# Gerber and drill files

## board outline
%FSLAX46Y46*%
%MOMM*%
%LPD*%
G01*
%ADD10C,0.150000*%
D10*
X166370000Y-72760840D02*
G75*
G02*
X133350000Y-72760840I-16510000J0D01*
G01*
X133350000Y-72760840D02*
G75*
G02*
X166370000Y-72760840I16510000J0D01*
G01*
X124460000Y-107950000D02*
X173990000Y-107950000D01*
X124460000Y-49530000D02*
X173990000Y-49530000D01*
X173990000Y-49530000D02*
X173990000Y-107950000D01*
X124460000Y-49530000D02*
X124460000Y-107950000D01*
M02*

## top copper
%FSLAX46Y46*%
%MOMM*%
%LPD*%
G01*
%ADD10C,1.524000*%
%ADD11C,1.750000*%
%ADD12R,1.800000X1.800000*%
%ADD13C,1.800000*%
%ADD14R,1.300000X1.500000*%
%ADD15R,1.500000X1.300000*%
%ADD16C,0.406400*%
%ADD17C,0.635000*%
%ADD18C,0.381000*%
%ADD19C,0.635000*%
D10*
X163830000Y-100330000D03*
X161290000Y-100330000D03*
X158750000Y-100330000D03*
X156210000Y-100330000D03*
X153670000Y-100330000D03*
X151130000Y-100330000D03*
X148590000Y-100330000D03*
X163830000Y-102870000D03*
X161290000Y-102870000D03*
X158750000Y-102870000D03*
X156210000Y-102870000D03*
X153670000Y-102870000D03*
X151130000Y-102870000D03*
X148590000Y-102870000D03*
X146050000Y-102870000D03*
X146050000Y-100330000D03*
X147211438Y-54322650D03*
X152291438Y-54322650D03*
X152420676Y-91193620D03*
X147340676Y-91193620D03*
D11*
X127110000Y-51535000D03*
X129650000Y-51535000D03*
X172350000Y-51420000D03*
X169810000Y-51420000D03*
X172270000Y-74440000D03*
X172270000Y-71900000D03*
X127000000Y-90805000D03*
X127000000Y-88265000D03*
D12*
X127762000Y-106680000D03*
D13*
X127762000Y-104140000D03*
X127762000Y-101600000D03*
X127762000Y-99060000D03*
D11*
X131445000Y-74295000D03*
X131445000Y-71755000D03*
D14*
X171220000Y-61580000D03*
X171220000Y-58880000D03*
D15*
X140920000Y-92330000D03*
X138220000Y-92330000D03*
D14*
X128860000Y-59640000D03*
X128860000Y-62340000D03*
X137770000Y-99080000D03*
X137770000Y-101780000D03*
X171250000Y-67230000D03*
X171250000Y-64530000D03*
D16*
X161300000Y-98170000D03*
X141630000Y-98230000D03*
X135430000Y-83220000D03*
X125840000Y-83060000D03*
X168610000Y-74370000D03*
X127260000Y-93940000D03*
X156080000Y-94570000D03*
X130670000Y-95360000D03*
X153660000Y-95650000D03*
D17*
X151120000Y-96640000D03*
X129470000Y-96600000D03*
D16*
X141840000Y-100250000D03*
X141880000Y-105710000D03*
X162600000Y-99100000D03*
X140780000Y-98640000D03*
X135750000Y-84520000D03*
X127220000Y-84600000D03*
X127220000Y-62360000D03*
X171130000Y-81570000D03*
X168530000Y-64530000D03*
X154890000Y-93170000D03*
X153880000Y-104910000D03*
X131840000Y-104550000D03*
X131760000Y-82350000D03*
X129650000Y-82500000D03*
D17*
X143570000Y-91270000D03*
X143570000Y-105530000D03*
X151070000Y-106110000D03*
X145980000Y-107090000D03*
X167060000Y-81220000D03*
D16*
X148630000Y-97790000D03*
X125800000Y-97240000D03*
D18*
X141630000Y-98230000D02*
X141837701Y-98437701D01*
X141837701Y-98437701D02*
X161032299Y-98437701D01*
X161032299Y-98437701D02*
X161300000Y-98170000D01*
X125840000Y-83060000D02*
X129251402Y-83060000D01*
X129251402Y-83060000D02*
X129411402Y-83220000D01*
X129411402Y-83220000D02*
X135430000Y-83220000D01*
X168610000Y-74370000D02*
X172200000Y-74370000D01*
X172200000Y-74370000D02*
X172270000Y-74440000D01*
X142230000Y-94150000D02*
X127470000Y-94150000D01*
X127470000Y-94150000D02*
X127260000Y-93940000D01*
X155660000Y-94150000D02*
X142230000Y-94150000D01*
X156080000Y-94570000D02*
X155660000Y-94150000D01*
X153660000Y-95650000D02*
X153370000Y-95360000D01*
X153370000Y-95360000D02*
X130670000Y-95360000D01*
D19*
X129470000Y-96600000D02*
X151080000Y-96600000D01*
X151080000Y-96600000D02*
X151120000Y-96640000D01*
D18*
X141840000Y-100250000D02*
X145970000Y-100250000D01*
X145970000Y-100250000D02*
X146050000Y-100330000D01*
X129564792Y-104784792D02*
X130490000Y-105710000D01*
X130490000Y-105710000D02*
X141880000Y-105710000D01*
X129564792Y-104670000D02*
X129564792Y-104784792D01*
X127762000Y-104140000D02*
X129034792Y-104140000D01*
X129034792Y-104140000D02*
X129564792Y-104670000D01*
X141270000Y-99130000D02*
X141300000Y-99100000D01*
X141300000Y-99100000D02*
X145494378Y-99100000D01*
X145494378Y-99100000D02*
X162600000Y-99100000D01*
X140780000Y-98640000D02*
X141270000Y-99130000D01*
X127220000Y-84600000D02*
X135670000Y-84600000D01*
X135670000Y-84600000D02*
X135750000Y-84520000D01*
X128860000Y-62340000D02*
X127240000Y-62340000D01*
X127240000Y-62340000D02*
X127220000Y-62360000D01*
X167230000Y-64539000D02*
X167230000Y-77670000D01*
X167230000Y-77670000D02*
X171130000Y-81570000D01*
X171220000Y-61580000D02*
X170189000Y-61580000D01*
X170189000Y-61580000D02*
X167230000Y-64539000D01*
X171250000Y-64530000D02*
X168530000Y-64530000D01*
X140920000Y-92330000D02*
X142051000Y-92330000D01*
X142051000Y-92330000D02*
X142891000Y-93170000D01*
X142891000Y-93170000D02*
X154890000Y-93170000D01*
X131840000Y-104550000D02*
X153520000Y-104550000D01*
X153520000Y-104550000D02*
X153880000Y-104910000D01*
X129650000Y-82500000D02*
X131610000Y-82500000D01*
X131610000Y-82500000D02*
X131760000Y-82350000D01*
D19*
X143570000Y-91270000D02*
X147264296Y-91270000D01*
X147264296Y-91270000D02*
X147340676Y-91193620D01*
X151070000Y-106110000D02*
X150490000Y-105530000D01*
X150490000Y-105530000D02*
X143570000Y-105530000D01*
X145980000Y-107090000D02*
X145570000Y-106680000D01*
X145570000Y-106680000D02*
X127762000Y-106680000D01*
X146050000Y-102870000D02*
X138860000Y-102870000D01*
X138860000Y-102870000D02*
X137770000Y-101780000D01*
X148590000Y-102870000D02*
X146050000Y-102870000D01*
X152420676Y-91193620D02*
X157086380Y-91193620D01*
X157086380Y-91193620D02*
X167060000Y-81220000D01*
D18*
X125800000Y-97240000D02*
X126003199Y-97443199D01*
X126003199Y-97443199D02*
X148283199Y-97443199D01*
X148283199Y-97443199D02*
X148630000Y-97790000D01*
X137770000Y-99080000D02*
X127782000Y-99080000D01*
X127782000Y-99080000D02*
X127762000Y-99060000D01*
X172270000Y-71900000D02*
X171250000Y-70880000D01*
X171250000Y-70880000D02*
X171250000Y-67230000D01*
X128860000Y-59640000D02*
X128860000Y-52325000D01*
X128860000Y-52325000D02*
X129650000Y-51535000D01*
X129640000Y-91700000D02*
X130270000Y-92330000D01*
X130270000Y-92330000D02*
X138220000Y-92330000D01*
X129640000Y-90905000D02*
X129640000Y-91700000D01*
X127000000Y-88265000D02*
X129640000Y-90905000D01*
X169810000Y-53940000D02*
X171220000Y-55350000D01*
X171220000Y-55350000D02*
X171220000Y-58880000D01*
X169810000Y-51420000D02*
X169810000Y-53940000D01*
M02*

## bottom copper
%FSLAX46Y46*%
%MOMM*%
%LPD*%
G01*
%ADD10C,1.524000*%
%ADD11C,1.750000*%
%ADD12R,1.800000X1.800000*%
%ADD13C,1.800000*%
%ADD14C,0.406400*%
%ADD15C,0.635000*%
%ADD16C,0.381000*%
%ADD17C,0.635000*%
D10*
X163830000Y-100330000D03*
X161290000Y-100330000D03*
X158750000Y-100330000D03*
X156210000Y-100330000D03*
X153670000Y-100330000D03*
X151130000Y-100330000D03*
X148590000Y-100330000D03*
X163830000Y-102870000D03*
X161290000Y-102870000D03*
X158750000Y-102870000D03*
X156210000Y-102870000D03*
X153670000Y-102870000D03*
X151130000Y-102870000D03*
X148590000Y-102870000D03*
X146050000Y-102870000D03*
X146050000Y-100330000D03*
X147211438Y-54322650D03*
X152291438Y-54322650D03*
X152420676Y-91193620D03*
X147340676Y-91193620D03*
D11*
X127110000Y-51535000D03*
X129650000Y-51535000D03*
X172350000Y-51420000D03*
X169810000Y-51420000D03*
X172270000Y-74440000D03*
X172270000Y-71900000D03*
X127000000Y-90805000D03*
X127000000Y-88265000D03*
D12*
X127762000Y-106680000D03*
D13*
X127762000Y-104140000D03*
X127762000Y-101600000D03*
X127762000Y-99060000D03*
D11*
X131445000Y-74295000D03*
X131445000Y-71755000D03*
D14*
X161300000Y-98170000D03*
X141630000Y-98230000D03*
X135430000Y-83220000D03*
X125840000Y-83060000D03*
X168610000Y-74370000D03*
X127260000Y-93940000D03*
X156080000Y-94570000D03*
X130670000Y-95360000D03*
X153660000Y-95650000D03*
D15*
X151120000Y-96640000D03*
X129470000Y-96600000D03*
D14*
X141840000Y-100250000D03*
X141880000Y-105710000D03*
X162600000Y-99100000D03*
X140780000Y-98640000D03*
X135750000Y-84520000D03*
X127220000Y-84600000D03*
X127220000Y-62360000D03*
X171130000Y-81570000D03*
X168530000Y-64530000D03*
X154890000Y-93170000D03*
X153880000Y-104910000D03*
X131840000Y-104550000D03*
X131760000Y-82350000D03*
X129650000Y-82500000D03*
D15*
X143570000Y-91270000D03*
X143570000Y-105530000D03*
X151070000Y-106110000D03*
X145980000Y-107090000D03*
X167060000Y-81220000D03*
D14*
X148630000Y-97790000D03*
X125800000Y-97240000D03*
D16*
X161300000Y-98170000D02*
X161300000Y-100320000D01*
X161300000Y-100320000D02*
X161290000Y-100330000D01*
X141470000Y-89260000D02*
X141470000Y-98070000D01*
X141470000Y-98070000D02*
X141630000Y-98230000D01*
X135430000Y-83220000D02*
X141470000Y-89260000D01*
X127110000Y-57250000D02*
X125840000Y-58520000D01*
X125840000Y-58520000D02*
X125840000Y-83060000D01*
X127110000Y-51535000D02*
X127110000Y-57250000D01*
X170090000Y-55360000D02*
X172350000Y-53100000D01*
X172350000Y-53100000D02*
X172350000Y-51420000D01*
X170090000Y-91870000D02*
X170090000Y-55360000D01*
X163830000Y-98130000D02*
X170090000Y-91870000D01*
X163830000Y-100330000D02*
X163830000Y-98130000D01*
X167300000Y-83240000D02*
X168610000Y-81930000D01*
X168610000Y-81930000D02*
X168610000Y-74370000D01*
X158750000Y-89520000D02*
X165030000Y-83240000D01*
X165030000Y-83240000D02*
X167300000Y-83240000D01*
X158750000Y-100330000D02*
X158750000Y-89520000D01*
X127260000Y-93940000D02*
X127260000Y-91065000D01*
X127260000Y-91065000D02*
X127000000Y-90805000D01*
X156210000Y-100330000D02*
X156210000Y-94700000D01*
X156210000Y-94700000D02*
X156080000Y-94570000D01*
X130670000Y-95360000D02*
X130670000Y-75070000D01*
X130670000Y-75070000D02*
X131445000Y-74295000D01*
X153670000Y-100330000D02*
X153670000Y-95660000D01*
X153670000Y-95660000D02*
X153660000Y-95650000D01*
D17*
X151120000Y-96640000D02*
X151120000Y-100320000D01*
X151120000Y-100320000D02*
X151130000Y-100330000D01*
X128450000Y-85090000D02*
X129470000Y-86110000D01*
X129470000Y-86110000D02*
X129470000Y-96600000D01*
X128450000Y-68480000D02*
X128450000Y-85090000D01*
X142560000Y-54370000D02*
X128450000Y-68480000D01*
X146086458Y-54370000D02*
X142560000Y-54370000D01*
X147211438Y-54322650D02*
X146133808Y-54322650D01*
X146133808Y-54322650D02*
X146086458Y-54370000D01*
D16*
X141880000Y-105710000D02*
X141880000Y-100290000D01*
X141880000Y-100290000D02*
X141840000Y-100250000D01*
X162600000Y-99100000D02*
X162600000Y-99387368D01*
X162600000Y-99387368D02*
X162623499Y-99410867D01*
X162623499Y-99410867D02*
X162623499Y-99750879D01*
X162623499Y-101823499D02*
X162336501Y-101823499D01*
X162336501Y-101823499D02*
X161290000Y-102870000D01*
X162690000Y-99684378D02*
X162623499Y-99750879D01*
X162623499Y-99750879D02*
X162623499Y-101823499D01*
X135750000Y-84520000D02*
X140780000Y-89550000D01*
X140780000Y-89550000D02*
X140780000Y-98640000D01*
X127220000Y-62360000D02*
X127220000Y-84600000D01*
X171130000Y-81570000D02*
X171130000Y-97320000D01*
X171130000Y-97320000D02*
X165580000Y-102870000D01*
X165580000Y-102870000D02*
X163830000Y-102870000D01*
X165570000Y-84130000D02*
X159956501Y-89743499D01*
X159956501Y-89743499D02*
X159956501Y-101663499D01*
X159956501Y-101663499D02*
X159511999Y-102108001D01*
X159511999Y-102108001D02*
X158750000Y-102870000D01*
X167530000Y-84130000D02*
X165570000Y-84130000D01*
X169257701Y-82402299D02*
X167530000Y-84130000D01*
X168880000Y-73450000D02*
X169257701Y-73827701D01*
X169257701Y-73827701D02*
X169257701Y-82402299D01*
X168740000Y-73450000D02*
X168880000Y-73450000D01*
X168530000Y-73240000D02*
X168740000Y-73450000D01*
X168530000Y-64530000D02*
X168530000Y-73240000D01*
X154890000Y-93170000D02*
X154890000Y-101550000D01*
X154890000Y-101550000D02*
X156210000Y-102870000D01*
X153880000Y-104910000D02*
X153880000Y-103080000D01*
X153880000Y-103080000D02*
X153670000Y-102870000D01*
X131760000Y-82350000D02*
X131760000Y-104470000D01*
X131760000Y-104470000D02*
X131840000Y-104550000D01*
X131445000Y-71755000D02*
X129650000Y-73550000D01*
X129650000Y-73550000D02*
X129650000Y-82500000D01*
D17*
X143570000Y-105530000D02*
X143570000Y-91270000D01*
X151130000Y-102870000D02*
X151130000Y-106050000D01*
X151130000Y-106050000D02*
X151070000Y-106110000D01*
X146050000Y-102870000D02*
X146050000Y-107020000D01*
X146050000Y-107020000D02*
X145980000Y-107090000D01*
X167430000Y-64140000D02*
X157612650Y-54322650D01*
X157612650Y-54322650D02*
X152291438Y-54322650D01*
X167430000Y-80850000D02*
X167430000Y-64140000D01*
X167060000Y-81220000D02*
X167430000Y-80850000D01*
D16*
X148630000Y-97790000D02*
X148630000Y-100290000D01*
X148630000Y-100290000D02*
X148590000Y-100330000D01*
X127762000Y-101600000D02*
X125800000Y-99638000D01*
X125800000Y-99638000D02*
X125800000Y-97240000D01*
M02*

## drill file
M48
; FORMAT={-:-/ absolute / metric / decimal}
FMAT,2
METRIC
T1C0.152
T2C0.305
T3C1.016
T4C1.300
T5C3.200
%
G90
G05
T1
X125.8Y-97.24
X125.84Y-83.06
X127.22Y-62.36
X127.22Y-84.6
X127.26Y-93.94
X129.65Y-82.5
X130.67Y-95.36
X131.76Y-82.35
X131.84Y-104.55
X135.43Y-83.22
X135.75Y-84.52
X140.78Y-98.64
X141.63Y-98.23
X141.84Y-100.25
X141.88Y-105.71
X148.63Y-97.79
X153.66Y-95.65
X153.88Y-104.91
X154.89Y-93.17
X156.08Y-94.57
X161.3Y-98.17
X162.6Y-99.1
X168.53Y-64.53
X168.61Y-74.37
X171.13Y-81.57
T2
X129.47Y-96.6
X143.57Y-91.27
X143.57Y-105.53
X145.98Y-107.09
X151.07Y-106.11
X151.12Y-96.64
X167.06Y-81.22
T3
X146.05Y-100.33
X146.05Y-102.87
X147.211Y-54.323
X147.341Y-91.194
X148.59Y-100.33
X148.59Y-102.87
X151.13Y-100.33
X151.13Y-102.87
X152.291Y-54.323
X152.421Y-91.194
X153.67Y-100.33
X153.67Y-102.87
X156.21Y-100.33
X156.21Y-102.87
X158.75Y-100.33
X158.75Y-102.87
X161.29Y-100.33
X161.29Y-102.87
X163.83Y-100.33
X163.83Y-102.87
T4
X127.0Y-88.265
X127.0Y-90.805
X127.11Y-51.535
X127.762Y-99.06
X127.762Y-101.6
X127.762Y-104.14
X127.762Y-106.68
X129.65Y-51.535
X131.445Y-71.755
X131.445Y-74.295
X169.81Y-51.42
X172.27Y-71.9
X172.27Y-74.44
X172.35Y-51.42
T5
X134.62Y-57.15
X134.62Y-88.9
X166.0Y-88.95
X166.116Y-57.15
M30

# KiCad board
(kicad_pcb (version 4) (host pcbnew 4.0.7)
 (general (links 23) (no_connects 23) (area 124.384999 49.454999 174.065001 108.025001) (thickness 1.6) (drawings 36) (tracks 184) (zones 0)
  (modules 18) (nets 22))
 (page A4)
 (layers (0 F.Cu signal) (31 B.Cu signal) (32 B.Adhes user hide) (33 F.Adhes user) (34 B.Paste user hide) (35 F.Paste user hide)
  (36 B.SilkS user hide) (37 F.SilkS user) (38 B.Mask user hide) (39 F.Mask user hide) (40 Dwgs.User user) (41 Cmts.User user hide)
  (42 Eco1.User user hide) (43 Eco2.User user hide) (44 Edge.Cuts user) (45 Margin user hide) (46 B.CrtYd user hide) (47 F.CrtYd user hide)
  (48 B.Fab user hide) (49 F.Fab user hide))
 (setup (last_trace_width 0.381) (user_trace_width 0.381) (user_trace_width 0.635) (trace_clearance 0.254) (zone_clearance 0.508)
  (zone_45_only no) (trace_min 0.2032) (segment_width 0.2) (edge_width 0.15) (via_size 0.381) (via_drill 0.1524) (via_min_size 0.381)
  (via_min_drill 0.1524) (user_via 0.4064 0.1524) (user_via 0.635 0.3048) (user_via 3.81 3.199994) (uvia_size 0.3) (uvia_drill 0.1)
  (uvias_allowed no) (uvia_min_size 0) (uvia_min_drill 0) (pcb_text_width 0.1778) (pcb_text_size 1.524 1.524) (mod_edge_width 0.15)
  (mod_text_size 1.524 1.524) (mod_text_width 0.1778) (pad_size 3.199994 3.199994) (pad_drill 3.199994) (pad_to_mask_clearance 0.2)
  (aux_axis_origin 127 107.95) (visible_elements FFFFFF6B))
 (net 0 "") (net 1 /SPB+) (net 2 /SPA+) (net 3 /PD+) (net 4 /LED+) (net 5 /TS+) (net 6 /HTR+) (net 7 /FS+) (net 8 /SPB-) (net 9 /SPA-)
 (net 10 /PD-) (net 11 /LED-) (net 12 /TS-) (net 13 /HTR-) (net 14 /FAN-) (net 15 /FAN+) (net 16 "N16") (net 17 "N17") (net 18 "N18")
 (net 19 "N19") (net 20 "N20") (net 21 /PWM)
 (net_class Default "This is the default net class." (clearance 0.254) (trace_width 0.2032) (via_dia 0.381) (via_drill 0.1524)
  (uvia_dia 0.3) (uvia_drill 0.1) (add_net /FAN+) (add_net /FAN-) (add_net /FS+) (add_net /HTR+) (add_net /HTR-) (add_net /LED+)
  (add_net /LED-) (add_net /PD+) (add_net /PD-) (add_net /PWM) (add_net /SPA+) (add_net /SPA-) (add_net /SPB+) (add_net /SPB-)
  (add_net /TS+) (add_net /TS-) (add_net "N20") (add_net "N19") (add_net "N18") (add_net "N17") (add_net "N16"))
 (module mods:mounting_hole (layer F.Cu) (at 166.116 57.15)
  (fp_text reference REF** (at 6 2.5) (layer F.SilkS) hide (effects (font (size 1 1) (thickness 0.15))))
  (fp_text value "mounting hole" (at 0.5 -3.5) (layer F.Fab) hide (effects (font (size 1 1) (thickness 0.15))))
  (pad "" np_thru_hole circle (at 0 0) (size 3.199994 3.199994) (drill 3.199994) (layers *.Cu *.Mask F.SilkS)))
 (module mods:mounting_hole (layer F.Cu) (at 134.62 88.9)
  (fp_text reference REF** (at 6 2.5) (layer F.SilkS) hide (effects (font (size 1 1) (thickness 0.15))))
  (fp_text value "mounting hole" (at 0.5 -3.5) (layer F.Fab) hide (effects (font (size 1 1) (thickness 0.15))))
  (pad "" np_thru_hole circle (at 0 0) (size 3.199994 3.199994) (drill 3.199994) (layers *.Cu *.Mask F.SilkS)))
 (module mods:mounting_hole (layer F.Cu) (at 134.62 57.15)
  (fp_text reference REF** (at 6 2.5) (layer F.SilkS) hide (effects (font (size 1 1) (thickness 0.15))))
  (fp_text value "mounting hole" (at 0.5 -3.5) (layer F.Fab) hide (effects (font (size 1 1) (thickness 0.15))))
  (pad "" np_thru_hole circle (at 0 0) (size 3.199994 3.199994) (drill 3.199994) (layers *.Cu *.Mask F.SilkS)))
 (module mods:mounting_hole (layer F.Cu) (at 165.999998 88.950013)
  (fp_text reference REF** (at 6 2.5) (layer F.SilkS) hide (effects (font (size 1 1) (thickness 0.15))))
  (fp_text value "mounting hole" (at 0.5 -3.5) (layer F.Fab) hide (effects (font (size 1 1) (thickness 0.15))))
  (pad "" np_thru_hole circle (at 0 0) (size 3.199994 3.199994) (drill 3.199994) (layers *.Cu *.Mask F.SilkS)))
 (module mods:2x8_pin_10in (layer F.Cu) (at 154.94 101.6 180)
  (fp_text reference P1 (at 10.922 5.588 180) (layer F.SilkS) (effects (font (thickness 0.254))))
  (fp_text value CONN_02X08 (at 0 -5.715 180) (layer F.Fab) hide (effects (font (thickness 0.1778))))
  (pad 1 thru_hole circle (at -8.89 1.27 180) (size 1.524 1.524) (drill 1.016) (layers *.Cu *.Mask F.SilkS) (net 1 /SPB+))
  (pad 3 thru_hole circle (at -6.35 1.27 180) (size 1.524 1.524) (drill 1.016) (layers *.Cu *.Mask F.SilkS) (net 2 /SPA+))
  (pad 5 thru_hole circle (at -3.81 1.27 180) (size 1.524 1.524) (drill 1.016) (layers *.Cu *.Mask F.SilkS) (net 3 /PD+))
  (pad 7 thru_hole circle (at -1.27 1.27 180) (size 1.524 1.524) (drill 1.016) (layers *.Cu *.Mask F.SilkS) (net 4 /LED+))
  (pad 9 thru_hole circle (at 1.27 1.27 180) (size 1.524 1.524) (drill 1.016) (layers *.Cu *.Mask F.SilkS) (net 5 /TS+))
  (pad 11 thru_hole circle (at 3.81 1.27 180) (size 1.524 1.524) (drill 1.016) (layers *.Cu *.Mask F.SilkS) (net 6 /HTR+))
  (pad 13 thru_hole circle (at 6.35 1.27 180) (size 1.524 1.524) (drill 1.016) (layers *.Cu *.Mask F.SilkS) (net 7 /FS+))
  (pad 2 thru_hole circle (at -8.89 -1.27 180) (size 1.524 1.524) (drill 1.016) (layers *.Cu *.Mask F.SilkS) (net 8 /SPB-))
  (pad 4 thru_hole circle (at -6.35 -1.27 180) (size 1.524 1.524) (drill 1.016) (layers *.Cu *.Mask F.SilkS) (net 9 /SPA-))
  (pad 6 thru_hole circle (at -3.81 -1.27 180) (size 1.524 1.524) (drill 1.016) (layers *.Cu *.Mask F.SilkS) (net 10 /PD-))
  (pad 8 thru_hole circle (at -1.27 -1.27 180) (size 1.524 1.524) (drill 1.016) (layers *.Cu *.Mask F.SilkS) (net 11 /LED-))
  (pad 10 thru_hole circle (at 1.27 -1.27 180) (size 1.524 1.524) (drill 1.016) (layers *.Cu *.Mask F.SilkS) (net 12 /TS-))
  (pad 12 thru_hole circle (at 3.81 -1.27 180) (size 1.524 1.524) (drill 1.016) (layers *.Cu *.Mask F.SilkS) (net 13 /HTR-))
  (pad 14 thru_hole circle (at 6.35 -1.27 180) (size 1.524 1.524) (drill 1.016) (layers *.Cu *.Mask F.SilkS) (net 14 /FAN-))
  (pad 16 thru_hole circle (at 8.89 -1.27 180) (size 1.524 1.524) (drill 1.016) (layers *.Cu *.Mask F.SilkS) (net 14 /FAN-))
  (pad 15 thru_hole circle (at 8.89 1.27 180) (size 1.524 1.524) (drill 1.016) (layers *.Cu *.Mask F.SilkS) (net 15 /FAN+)))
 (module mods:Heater (layer F.Cu) (at 149.751438 54.32265)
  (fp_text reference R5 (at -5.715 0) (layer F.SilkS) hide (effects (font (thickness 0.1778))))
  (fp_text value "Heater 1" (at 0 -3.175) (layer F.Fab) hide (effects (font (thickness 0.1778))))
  (pad 1 thru_hole circle (at -2.54 0) (size 1.524 1.524) (drill 1.016) (layers *.Cu *.Mask F.SilkS) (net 6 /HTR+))
  (pad 2 thru_hole circle (at 2.54 0) (size 1.524 1.524) (drill 1.016) (layers *.Cu *.Mask F.SilkS) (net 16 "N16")))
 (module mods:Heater (layer F.Cu) (at 149.880676 91.19362 180)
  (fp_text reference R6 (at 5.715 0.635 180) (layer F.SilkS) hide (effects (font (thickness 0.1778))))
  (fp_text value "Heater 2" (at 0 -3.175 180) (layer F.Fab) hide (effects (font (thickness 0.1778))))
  (pad 1 thru_hole circle (at -2.54 0 180) (size 1.524 1.524) (drill 1.016) (layers *.Cu *.Mask F.SilkS) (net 16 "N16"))
  (pad 2 thru_hole circle (at 2.54 0 180) (size 1.524 1.524) (drill 1.016) (layers *.Cu *.Mask F.SilkS) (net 13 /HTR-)))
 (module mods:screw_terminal (layer F.Cu) (at 128.38 51.535)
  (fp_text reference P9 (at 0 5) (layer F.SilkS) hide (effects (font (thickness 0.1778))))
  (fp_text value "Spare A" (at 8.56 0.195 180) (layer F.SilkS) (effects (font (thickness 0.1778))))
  (pad 1 thru_hole circle (at -1.27 0) (size 1.75 1.75) (drill 1.3) (layers *.Cu *.Mask F.SilkS) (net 2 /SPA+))
  (pad 2 thru_hole circle (at 1.27 0) (size 1.75 1.75) (drill 1.3) (layers *.Cu *.Mask F.SilkS) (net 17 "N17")))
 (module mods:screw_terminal (layer F.Cu) (at 171.08 51.42 180)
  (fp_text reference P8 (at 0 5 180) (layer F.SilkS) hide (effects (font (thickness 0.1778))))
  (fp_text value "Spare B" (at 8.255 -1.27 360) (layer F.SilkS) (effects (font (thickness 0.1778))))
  (pad 1 thru_hole circle (at -1.27 0 180) (size 1.75 1.75) (drill 1.3) (layers *.Cu *.Mask F.SilkS) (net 1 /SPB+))
  (pad 2 thru_hole circle (at 1.27 0 180) (size 1.75 1.75) (drill 1.3) (layers *.Cu *.Mask F.SilkS) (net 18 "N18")))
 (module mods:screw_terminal (layer F.Cu) (at 172.27 73.17 90)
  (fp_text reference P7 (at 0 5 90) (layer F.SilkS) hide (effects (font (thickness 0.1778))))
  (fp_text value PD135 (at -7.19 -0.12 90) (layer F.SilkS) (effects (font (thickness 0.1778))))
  (pad 1 thru_hole circle (at -1.27 0 90) (size 1.75 1.75) (drill 1.3) (layers *.Cu *.Mask F.SilkS) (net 3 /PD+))
  (pad 2 thru_hole circle (at 1.27 0 90) (size 1.75 1.75) (drill 1.3) (layers *.Cu *.Mask F.SilkS) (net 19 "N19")))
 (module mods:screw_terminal (layer F.Cu) (at 127 89.535 90)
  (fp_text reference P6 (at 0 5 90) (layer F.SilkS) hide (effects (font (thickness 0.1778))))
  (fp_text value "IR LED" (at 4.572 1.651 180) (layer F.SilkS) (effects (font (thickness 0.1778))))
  (pad 1 thru_hole circle (at -1.27 0 90) (size 1.75 1.75) (drill 1.3) (layers *.Cu *.Mask F.SilkS) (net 4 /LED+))
  (pad 2 thru_hole circle (at 1.27 0 90) (size 1.75 1.75) (drill 1.3) (layers *.Cu *.Mask F.SilkS) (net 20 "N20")))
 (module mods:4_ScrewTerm (layer F.Cu) (at 127.762 102.87 90)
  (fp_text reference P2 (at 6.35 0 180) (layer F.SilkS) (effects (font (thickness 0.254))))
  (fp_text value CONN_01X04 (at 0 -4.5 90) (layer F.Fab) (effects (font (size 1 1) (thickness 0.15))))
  (pad 1 thru_hole rect (at -3.81 0 90) (size 1.8 1.8) (drill 1.3) (layers *.Cu *.Mask) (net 14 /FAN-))
  (pad 2 thru_hole circle (at -1.27 0 90) (size 1.8 1.8) (drill 1.3) (layers *.Cu *.Mask) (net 15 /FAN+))
  (pad 3 thru_hole circle (at 1.27 0 90) (size 1.8 1.8) (drill 1.3) (layers *.Cu *.Mask) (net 7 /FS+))
  (pad 4 thru_hole circle (at 3.81 0 90) (size 1.8 1.8) (drill 1.3) (layers *.Cu *.Mask) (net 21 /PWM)))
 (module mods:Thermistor (layer F.Cu) (at 131.445 73.025 90)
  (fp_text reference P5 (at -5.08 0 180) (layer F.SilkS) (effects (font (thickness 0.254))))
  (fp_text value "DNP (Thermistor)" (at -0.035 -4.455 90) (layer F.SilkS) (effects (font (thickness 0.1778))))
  (pad 1 thru_hole circle (at -1.27 0 90) (size 1.75 1.75) (drill 1.3) (layers *.Cu *.Mask F.SilkS) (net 5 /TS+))
  (pad 2 thru_hole circle (at 1.27 0 90) (size 1.75 1.75) (drill 1.3) (layers *.Cu *.Mask F.SilkS) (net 12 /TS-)))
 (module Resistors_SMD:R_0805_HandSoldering (layer F.Cu) (at 171.22 60.23 90)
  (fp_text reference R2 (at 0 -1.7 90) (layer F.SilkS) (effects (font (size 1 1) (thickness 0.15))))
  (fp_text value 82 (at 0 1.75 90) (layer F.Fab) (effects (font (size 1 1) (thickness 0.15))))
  (pad 1 smd rect (at -1.35 0 90) (size 1.5 1.3) (layers F.Cu F.Paste F.Mask) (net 8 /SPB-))
  (pad 2 smd rect (at 1.35 0 90) (size 1.5 1.3) (layers F.Cu F.Paste F.Mask) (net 18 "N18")))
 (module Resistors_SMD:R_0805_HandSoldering (layer F.Cu) (at 139.57 92.33 180)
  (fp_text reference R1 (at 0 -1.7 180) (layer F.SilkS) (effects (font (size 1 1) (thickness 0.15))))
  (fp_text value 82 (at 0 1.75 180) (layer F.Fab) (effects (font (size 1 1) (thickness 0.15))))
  (pad 1 smd rect (at -1.35 0 180) (size 1.5 1.3) (layers F.Cu F.Paste F.Mask) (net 11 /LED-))
  (pad 2 smd rect (at 1.35 0 180) (size 1.5 1.3) (layers F.Cu F.Paste F.Mask) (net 20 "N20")))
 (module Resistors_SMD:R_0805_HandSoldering (layer F.Cu) (at 128.86 60.99 270)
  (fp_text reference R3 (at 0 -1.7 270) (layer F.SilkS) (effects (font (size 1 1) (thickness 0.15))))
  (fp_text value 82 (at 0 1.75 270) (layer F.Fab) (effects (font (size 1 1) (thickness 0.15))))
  (pad 1 smd rect (at -1.35 0 270) (size 1.5 1.3) (layers F.Cu F.Paste F.Mask) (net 17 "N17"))
  (pad 2 smd rect (at 1.35 0 270) (size 1.5 1.3) (layers F.Cu F.Paste F.Mask) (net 9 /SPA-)))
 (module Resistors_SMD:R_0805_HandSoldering (layer F.Cu) (at 137.77 100.43 270)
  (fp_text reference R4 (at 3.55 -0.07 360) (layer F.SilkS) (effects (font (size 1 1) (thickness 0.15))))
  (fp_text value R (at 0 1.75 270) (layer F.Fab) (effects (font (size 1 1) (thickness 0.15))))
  (pad 1 smd rect (at -1.35 0 270) (size 1.5 1.3) (layers F.Cu F.Paste F.Mask) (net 21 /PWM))
  (pad 2 smd rect (at 1.35 0 270) (size 1.5 1.3) (layers F.Cu F.Paste F.Mask) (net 14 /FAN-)))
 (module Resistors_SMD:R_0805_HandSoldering (layer F.Cu) (at 171.25 65.88 90)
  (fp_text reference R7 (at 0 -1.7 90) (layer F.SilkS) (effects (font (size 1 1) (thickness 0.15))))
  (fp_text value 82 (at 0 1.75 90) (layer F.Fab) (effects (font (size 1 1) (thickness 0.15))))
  (pad 1 smd rect (at -1.35 0 90) (size 1.5 1.3) (layers F.Cu F.Paste F.Mask) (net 19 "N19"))
  (pad 2 smd rect (at 1.35 0 90) (size 1.5 1.3) (layers F.Cu F.Paste F.Mask) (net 10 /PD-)))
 (gr_circle (center 149.86 72.76084) (end 133.35 72.76084) (layer Edge.Cuts) (width 0.15))
 (gr_line (start 124.46 107.95) (end 173.99 107.95) (angle 90) (layer Edge.Cuts) (width 0.15))
 (gr_line (start 124.46 49.53) (end 173.99 49.53) (angle 90) (layer Edge.Cuts) (width 0.15))
 (gr_line (start 173.99 49.53) (end 173.99 107.95) (angle 90) (layer Edge.Cuts) (width 0.15))
 (gr_line (start 124.46 49.53) (end 124.46 107.95) (angle 90) (layer Edge.Cuts) (width 0.15))
 (segment (start 161.3 98.17) (end 161.3 100.32) (width 0.381) (layer B.Cu) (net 2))
 (segment (start 161.3 100.32) (end 161.29 100.33) (width 0.381) (layer B.Cu) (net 2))
 (segment (start 141.63 98.23) (end 141.837701 98.437701) (width 0.381) (layer F.Cu) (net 2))
 (segment (start 141.837701 98.437701) (end 161.032299 98.437701) (width 0.381) (layer F.Cu) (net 2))
 (via (at 161.3 98.17) (size 0.4064) (drill 0.1524) (layers F.Cu B.Cu) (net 2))
 (segment (start 161.032299 98.437701) (end 161.3 98.17) (width 0.381) (layer F.Cu) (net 2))
 (segment (start 141.47 89.26) (end 141.47 98.07) (width 0.381) (layer B.Cu) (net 2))
 (via (at 141.63 98.23) (size 0.4064) (drill 0.1524) (layers F.Cu B.Cu) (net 2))
 (segment (start 141.47 98.07) (end 141.63 98.23) (width 0.381) (layer B.Cu) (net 2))
 (segment (start 135.43 83.22) (end 141.47 89.26) (width 0.381) (layer B.Cu) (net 2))
 (segment (start 125.84 83.06) (end 129.251402 83.06) (width 0.381) (layer F.Cu) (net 2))
 (segment (start 129.251402 83.06) (end 129.411402 83.22) (width 0.381) (layer F.Cu) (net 2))
 (segment (start 129.411402 83.22) (end 135.43 83.22) (width 0.381) (layer F.Cu) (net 2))
 (via (at 135.43 83.22) (size 0.4064) (drill 0.1524) (layers F.Cu B.Cu) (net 2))
 (segment (start 127.11 57.25) (end 125.84 58.52) (width 0.381) (layer B.Cu) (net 2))
 (via (at 125.84 83.06) (size 0.4064) (drill 0.1524) (layers F.Cu B.Cu) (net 2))
 (segment (start 125.84 58.52) (end 125.84 83.06) (width 0.381) (layer B.Cu) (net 2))
 (segment (start 127.11 51.535) (end 127.11 57.25) (width 0.381) (layer B.Cu) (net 2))
 (segment (start 170.09 55.36) (end 172.35 53.1) (width 0.381) (layer B.Cu) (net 1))
 (segment (start 172.35 53.1) (end 172.35 51.42) (width 0.381) (layer B.Cu) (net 1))
 (segment (start 170.09 91.87) (end 170.09 55.36) (width 0.381) (layer B.Cu) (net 1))
 (segment (start 163.83 98.13) (end 170.09 91.87) (width 0.381) (layer B.Cu) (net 1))
 (segment (start 163.83 100.33) (end 163.83 98.13) (width 0.381) (layer B.Cu) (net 1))
 (segment (start 168.61 74.37) (end 172.2 74.37) (width 0.381) (layer F.Cu) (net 3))
 (segment (start 172.2 74.37) (end 172.27 74.44) (width 0.381) (layer F.Cu) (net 3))
 (segment (start 167.3 83.24) (end 168.61 81.93) (width 0.381) (layer B.Cu) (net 3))
 (segment (start 168.61 81.93) (end 168.61 74.37) (width 0.381) (layer B.Cu) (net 3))
 (via (at 168.61 74.37) (size 0.4064) (drill 0.1524) (layers F.Cu B.Cu) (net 3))
 (segment (start 158.75 89.52) (end 165.03 83.24) (width 0.381) (layer B.Cu) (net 3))
 (segment (start 165.03 83.24) (end 167.3 83.24) (width 0.381) (layer B.Cu) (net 3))
 (segment (start 158.75 100.33) (end 158.75 89.52) (width 0.381) (layer B.Cu) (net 3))
 (segment (start 127.26 93.94) (end 127.26 91.065) (width 0.381) (layer B.Cu) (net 4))
 (segment (start 127.26 91.065) (end 127 90.805) (width 0.381) (layer B.Cu) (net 4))
 (segment (start 142.23 94.15) (end 127.47 94.15) (width 0.381) (layer F.Cu) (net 4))
 (segment (start 127.47 94.15) (end 127.26 93.94) (width 0.381) (layer F.Cu) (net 4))
 (via (at 127.26 93.94) (size 0.4064) (drill 0.1524) (layers F.Cu B.Cu) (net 4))
 (segment (start 155.66 94.15) (end 142.23 94.15) (width 0.381) (layer F.Cu) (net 4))
 (segment (start 156.08 94.57) (end 155.66 94.15) (width 0.381) (layer F.Cu) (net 4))
 (segment (start 156.21 100.33) (end 156.21 94.7) (width 0.381) (layer B.Cu) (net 4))
 (segment (start 156.21 94.7) (end 156.08 94.57) (width 0.381) (layer B.Cu) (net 4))
 (via (at 156.08 94.57) (size 0.4064) (drill 0.1524) (layers F.Cu B.Cu) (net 4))
 (segment (start 130.67 95.36) (end 130.67 75.07) (width 0.381) (layer B.Cu) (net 5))
 (segment (start 130.67 75.07) (end 131.445 74.295) (width 0.381) (layer B.Cu) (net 5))
 (segment (start 153.66 95.65) (end 153.37 95.36) (width 0.381) (layer F.Cu) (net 5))
 (segment (start 153.37 95.36) (end 130.67 95.36) (width 0.381) (layer F.Cu) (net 5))
 (via (at 130.67 95.36) (size 0.4064) (drill 0.1524) (layers F.Cu B.Cu) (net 5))
 (segment (start 153.67 100.33) (end 153.67 95.66) (width 0.381) (layer B.Cu) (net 5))
 (segment (start 153.67 95.66) (end 153.66 95.65) (width 0.381) (layer B.Cu) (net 5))
 (via (at 153.66 95.65) (size 0.4064) (drill 0.1524) (layers F.Cu B.Cu) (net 5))
 (segment (start 151.12 96.64) (end 151.12 100.32) (width 0.635) (layer B.Cu) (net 6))
 (segment (start 151.12 100.32) (end 151.13 100.33) (width 0.635) (layer B.Cu) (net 6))
 (segment (start 129.47 96.6) (end 151.08 96.6) (width 0.635) (layer F.Cu) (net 6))
 (segment (start 151.08 96.6) (end 151.12 96.64) (width 0.635) (layer F.Cu) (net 6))
 (via (at 151.12 96.64) (size 0.635) (drill 0.3048) (layers F.Cu B.Cu) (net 6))
 (segment (start 128.45 85.09) (end 129.47 86.11) (width 0.635) (layer B.Cu) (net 6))
 (segment (start 129.47 86.11) (end 129.47 96.6) (width 0.635) (layer B.Cu) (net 6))
 (via (at 129.47 96.6) (size 0.635) (drill 0.3048) (layers F.Cu B.Cu) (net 6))
 (segment (start 128.45 68.48) (end 128.45 85.09) (width 0.635) (layer B.Cu) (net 6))
 (segment (start 142.56 54.37) (end 128.45 68.48) (width 0.635) (layer B.Cu) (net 6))
 (segment (start 146.086458 54.37) (end 142.56 54.37) (width 0.635) (layer B.Cu) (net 6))
 (segment (start 147.211438 54.32265) (end 146.133808 54.32265) (width 0.635) (layer B.Cu) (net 6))
 (segment (start 146.133808 54.32265) (end 146.086458 54.37) (width 0.635) (layer B.Cu) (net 6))
 (segment (start 141.84 100.25) (end 145.97 100.25) (width 0.381) (layer F.Cu) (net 15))
 (segment (start 145.97 100.25) (end 146.05 100.33) (width 0.381) (layer F.Cu) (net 15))
 (segment (start 141.88 105.71) (end 141.88 100.29) (width 0.381) (layer B.Cu) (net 15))
 (segment (start 141.88 100.29) (end 141.84 100.25) (width 0.381) (layer B.Cu) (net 15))
 (via (at 141.84 100.25) (size 0.4064) (drill 0.1524) (layers F.Cu B.Cu) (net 15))
 (segment (start 129.564792 104.784792) (end 130.49 105.71) (width 0.381) (layer F.Cu) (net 15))
 (segment (start 130.49 105.71) (end 141.88 105.71) (width 0.381) (layer F.Cu) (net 15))
 (via (at 141.88 105.71) (size 0.4064) (drill 0.1524) (layers F.Cu B.Cu) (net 15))
 (segment (start 129.564792 104.67) (end 129.564792 104.784792) (width 0.381) (layer F.Cu) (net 15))
 (segment (start 127.762 104.14) (end 129.034792 104.14) (width 0.381) (layer F.Cu) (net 15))
 (segment (start 129.034792 104.14) (end 129.564792 104.67) (width 0.381) (layer F.Cu) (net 15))
 (segment (start 162.6 99.1) (end 162.6 99.387368) (width 0.381) (layer B.Cu) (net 9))
 (segment (start 162.6 99.387368) (end 162.623499 99.410867) (width 0.381) (layer B.Cu) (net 9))
 (segment (start 162.623499 99.410867) (end 162.623499 99.750879) (width 0.381) (layer B.Cu) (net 9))
 (segment (start 141.27 99.13) (end 141.3 99.1) (width 0.381) (layer F.Cu) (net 9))
 (segment (start 141.3 99.1) (end 145.494378 99.1) (width 0.381) (layer F.Cu) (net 9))
 (segment (start 145.494378 99.1) (end 162.6 99.1) (width 0.381) (layer F.Cu) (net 9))
 (via (at 162.6 99.1) (size 0.4064) (drill 0.1524) (layers F.Cu B.Cu) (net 9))
 (segment (start 140.78 98.64) (end 141.27 99.13) (width 0.381) (layer F.Cu) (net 9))
 (segment (start 162.623499 101.823499) (end 162.336501 101.823499) (width 0.381) (layer B.Cu) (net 9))
 (segment (start 162.336501 101.823499) (end 161.29 102.87) (width 0.381) (layer B.Cu) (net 9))
 (segment (start 162.69 99.684378) (end 162.623499 99.750879) (width 0.381) (layer B.Cu) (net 9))
 (segment (start 162.623499 99.750879) (end 162.623499 101.823499) (width 0.381) (layer B.Cu) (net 9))
 (segment (start 135.75 84.52) (end 140.78 89.55) (width 0.381) (layer B.Cu) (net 9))
 (segment (start 140.78 89.55) (end 140.78 98.64) (width 0.381) (layer B.Cu) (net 9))
 (via (at 140.78 98.64) (size 0.4064) (drill 0.1524) (layers F.Cu B.Cu) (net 9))
 (segment (start 127.22 84.6) (end 135.67 84.6) (width 0.381) (layer F.Cu) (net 9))
 (segment (start 135.67 84.6) (end 135.75 84.52) (width 0.381) (layer F.Cu) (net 9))
 (via (at 135.75 84.52) (size 0.4064) (drill 0.1524) (layers F.Cu B.Cu) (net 9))
 (segment (start 127.22 62.36) (end 127.22 84.6) (width 0.381) (layer B.Cu) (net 9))
 (via (at 127.22 84.6) (size 0.4064) (drill 0.1524) (layers F.Cu B.Cu) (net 9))
 (segment (start 128.86 62.34) (end 127.24 62.34) (width 0.381) (layer F.Cu) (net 9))
 (segment (start 127.24 62.34) (end 127.22 62.36) (width 0.381) (layer F.Cu) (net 9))
 (via (at 127.22 62.36) (size 0.4064) (drill 0.1524) (layers F.Cu B.Cu) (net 9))
 (segment (start 171.13 81.57) (end 171.13 97.32) (width 0.381) (layer B.Cu) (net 8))
 (segment (start 171.13 97.32) (end 165.58 102.87) (width 0.381) (layer B.Cu) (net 8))
 (segment (start 165.58 102.87) (end 163.83 102.87) (width 0.381) (layer B.Cu) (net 8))
 (segment (start 167.23 64.539) (end 167.23 77.67) (width 0.381) (layer F.Cu) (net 8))
 (segment (start 167.23 77.67) (end 171.13 81.57) (width 0.381) (layer F.Cu) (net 8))
 (via (at 171.13 81.57) (size 0.4064) (drill 0.1524) (layers F.Cu B.Cu) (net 8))
 (segment (start 171.22 61.58) (end 170.189 61.58) (width 0.381) (layer F.Cu) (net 8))
 (segment (start 170.189 61.58) (end 167.23 64.539) (width 0.381) (layer F.Cu) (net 8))
 (segment (start 165.57 84.13) (end 159.956501 89.743499) (width 0.381) (layer B.Cu) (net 10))
 (segment (start 159.956501 89.743499) (end 159.956501 101.663499) (width 0.381) (layer B.Cu) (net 10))
 (segment (start 159.956501 101.663499) (end 159.511999 102.108001) (width 0.381) (layer B.Cu) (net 10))
 (segment (start 159.511999 102.108001) (end 158.75 102.87) (width 0.381) (layer B.Cu) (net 10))
 (segment (start 167.53 84.13) (end 165.57 84.13) (width 0.381) (layer B.Cu) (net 10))
 (segment (start 169.257701 82.402299) (end 167.53 84.13) (width 0.381) (layer B.Cu) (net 10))
 (segment (start 168.88 73.45) (end 169.257701 73.827701) (width 0.381) (layer B.Cu) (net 10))
 (segment (start 169.257701 73.827701) (end 169.257701 82.402299) (width 0.381) (layer B.Cu) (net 10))
 (segment (start 168.74 73.45) (end 168.88 73.45) (width 0.381) (layer B.Cu) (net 10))
 (segment (start 168.53 73.24) (end 168.74 73.45) (width 0.381) (layer B.Cu) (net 10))
 (segment (start 168.53 64.53) (end 168.53 73.24) (width 0.381) (layer B.Cu) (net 10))
 (segment (start 171.25 64.53) (end 168.53 64.53) (width 0.381) (layer F.Cu) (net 10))
 (via (at 168.53 64.53) (size 0.4064) (drill 0.1524) (layers F.Cu B.Cu) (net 10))
 (segment (start 154.89 93.17) (end 154.89 101.55) (width 0.381) (layer B.Cu) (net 11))
 (segment (start 154.89 101.55) (end 156.21 102.87) (width 0.381) (layer B.Cu) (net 11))
 (segment (start 140.92 92.33) (end 142.051 92.33) (width 0.381) (layer F.Cu) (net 11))
 (segment (start 142.051 92.33) (end 142.891 93.17) (width 0.381) (layer F.Cu) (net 11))
 (segment (start 142.891 93.17) (end 154.89 93.17) (width 0.381) (layer F.Cu) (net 11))
 (via (at 154.89 93.17) (size 0.4064) (drill 0.1524) (layers F.Cu B.Cu) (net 11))
 (segment (start 153.88 104.91) (end 153.88 103.08) (width 0.381) (layer B.Cu) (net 12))
 (segment (start 153.88 103.08) (end 153.67 102.87) (width 0.381) (layer B.Cu) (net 12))
 (segment (start 131.84 104.55) (end 153.52 104.55) (width 0.381) (layer F.Cu) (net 12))
 (segment (start 153.52 104.55) (end 153.88 104.91) (width 0.381) (layer F.Cu) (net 12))
 (via (at 153.88 104.91) (size 0.4064) (drill 0.1524) (layers F.Cu B.Cu) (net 12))
 (segment (start 131.76 82.35) (end 131.76 104.47) (width 0.381) (layer B.Cu) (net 12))
 (segment (start 131.76 104.47) (end 131.84 104.55) (width 0.381) (layer B.Cu) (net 12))
 (via (at 131.84 104.55) (size 0.4064) (drill 0.1524) (layers F.Cu B.Cu) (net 12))
 (segment (start 129.65 82.5) (end 131.61 82.5) (width 0.381) (layer F.Cu) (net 12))
 (segment (start 131.61 82.5) (end 131.76 82.35) (width 0.381) (layer F.Cu) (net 12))
 (via (at 131.76 82.35) (size 0.4064) (drill 0.1524) (layers F.Cu B.Cu) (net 12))
 (segment (start 131.445 71.755) (end 129.65 73.55) (width 0.381) (layer B.Cu) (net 12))
 (segment (start 129.65 73.55) (end 129.65 82.5) (width 0.381) (layer B.Cu) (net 12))
 (via (at 129.65 82.5) (size 0.4064) (drill 0.1524) (layers F.Cu B.Cu) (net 12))
 (segment (start 143.57 91.27) (end 147.264296 91.27) (width 0.635) (layer F.Cu) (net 13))
 (segment (start 147.264296 91.27) (end 147.340676 91.19362) (width 0.635) (layer F.Cu) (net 13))
 (segment (start 143.57 105.53) (end 143.57 91.27) (width 0.635) (layer B.Cu) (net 13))
 (via (at 143.57 91.27) (size 0.635) (drill 0.3048) (layers F.Cu B.Cu) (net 13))
 (segment (start 151.07 106.11) (end 150.49 105.53) (width 0.635) (layer F.Cu) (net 13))
 (segment (start 150.49 105.53) (end 143.57 105.53) (width 0.635) (layer F.Cu) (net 13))
 (via (at 143.57 105.53) (size 0.635) (drill 0.3048) (layers F.Cu B.Cu) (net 13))
 (segment (start 151.13 102.87) (end 151.13 106.05) (width 0.635) (layer B.Cu) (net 13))
 (segment (start 151.13 106.05) (end 151.07 106.11) (width 0.635) (layer B.Cu) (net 13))
 (via (at 151.07 106.11) (size 0.635) (drill 0.3048) (layers F.Cu B.Cu) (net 13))
 (segment (start 145.98 107.09) (end 145.57 106.68) (width 0.635) (layer F.Cu) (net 14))
 (segment (start 145.57 106.68) (end 127.762 106.68) (width 0.635) (layer F.Cu) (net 14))
 (segment (start 146.05 102.87) (end 146.05 107.02) (width 0.635) (layer B.Cu) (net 14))
 (segment (start 146.05 107.02) (end 145.98 107.09) (width 0.635) (layer B.Cu) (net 14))
 (via (at 145.98 107.09) (size 0.635) (drill 0.3048) (layers F.Cu B.Cu) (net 14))
 (segment (start 146.05 102.87) (end 138.86 102.87) (width 0.635) (layer F.Cu) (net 14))
 (segment (start 138.86 102.87) (end 137.77 101.78) (width 0.635) (layer F.Cu) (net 14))
 (segment (start 148.59 102.87) (end 146.05 102.87) (width 0.635) (layer F.Cu) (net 14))
 (segment (start 167.43 64.14) (end 157.61265 54.32265) (width 0.635) (layer B.Cu) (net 16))
 (segment (start 157.61265 54.32265) (end 152.291438 54.32265) (width 0.635) (layer B.Cu) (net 16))
 (segment (start 167.43 80.85) (end 167.43 64.14) (width 0.635) (layer B.Cu) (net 16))
 (segment (start 167.06 81.22) (end 167.43 80.85) (width 0.635) (layer B.Cu) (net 16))
 (segment (start 152.420676 91.19362) (end 157.08638 91.19362) (width 0.635) (layer F.Cu) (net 16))
 (segment (start 157.08638 91.19362) (end 167.06 81.22) (width 0.635) (layer F.Cu) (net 16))
 (via (at 167.06 81.22) (size 0.635) (drill 0.3048) (layers F.Cu B.Cu) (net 16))
 (segment (start 148.63 97.79) (end 148.63 100.29) (width 0.381) (layer B.Cu) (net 7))
 (segment (start 148.63 100.29) (end 148.59 100.33) (width 0.381) (layer B.Cu) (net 7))
 (segment (start 125.8 97.24) (end 126.003199 97.443199) (width 0.381) (layer F.Cu) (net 7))
 (segment (start 126.003199 97.443199) (end 148.283199 97.443199) (width 0.381) (layer F.Cu) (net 7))
 (via (at 148.63 97.79) (size 0.4064) (drill 0.1524) (layers F.Cu B.Cu) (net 7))
 (segment (start 148.283199 97.443199) (end 148.63 97.79) (width 0.381) (layer F.Cu) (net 7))
 (segment (start 127.762 101.6) (end 125.8 99.638) (width 0.381) (layer B.Cu) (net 7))
 (segment (start 125.8 99.638) (end 125.8 97.24) (width 0.381) (layer B.Cu) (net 7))
 (via (at 125.8 97.24) (size 0.4064) (drill 0.1524) (layers F.Cu B.Cu) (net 7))
 (segment (start 137.77 99.08) (end 127.782 99.08) (width 0.381) (layer F.Cu) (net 21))
 (segment (start 127.782 99.08) (end 127.762 99.06) (width 0.381) (layer F.Cu) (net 21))
 (segment (start 172.27 71.9) (end 171.25 70.88) (width 0.381) (layer F.Cu) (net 19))
 (segment (start 171.25 70.88) (end 171.25 67.23) (width 0.381) (layer F.Cu) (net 19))
 (segment (start 128.86 59.64) (end 128.86 52.325) (width 0.381) (layer F.Cu) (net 17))
 (segment (start 128.86 52.325) (end 129.65 51.535) (width 0.381) (layer F.Cu) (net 17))
 (segment (start 129.64 91.7) (end 130.27 92.33) (width 0.381) (layer F.Cu) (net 20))
 (segment (start 130.27 92.33) (end 138.22 92.33) (width 0.381) (layer F.Cu) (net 20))
 (segment (start 129.64 90.905) (end 129.64 91.7) (width 0.381) (layer F.Cu) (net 20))
 (segment (start 127 88.265) (end 129.64 90.905) (width 0.381) (layer F.Cu) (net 20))
 (segment (start 169.81 53.94) (end 171.22 55.35) (width 0.381) (layer F.Cu) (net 18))
 (segment (start 171.22 55.35) (end 171.22 58.88) (width 0.381) (layer F.Cu) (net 18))
 (segment (start 169.81 51.42) (end 169.81 53.94) (width 0.381) (layer F.Cu) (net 18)))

